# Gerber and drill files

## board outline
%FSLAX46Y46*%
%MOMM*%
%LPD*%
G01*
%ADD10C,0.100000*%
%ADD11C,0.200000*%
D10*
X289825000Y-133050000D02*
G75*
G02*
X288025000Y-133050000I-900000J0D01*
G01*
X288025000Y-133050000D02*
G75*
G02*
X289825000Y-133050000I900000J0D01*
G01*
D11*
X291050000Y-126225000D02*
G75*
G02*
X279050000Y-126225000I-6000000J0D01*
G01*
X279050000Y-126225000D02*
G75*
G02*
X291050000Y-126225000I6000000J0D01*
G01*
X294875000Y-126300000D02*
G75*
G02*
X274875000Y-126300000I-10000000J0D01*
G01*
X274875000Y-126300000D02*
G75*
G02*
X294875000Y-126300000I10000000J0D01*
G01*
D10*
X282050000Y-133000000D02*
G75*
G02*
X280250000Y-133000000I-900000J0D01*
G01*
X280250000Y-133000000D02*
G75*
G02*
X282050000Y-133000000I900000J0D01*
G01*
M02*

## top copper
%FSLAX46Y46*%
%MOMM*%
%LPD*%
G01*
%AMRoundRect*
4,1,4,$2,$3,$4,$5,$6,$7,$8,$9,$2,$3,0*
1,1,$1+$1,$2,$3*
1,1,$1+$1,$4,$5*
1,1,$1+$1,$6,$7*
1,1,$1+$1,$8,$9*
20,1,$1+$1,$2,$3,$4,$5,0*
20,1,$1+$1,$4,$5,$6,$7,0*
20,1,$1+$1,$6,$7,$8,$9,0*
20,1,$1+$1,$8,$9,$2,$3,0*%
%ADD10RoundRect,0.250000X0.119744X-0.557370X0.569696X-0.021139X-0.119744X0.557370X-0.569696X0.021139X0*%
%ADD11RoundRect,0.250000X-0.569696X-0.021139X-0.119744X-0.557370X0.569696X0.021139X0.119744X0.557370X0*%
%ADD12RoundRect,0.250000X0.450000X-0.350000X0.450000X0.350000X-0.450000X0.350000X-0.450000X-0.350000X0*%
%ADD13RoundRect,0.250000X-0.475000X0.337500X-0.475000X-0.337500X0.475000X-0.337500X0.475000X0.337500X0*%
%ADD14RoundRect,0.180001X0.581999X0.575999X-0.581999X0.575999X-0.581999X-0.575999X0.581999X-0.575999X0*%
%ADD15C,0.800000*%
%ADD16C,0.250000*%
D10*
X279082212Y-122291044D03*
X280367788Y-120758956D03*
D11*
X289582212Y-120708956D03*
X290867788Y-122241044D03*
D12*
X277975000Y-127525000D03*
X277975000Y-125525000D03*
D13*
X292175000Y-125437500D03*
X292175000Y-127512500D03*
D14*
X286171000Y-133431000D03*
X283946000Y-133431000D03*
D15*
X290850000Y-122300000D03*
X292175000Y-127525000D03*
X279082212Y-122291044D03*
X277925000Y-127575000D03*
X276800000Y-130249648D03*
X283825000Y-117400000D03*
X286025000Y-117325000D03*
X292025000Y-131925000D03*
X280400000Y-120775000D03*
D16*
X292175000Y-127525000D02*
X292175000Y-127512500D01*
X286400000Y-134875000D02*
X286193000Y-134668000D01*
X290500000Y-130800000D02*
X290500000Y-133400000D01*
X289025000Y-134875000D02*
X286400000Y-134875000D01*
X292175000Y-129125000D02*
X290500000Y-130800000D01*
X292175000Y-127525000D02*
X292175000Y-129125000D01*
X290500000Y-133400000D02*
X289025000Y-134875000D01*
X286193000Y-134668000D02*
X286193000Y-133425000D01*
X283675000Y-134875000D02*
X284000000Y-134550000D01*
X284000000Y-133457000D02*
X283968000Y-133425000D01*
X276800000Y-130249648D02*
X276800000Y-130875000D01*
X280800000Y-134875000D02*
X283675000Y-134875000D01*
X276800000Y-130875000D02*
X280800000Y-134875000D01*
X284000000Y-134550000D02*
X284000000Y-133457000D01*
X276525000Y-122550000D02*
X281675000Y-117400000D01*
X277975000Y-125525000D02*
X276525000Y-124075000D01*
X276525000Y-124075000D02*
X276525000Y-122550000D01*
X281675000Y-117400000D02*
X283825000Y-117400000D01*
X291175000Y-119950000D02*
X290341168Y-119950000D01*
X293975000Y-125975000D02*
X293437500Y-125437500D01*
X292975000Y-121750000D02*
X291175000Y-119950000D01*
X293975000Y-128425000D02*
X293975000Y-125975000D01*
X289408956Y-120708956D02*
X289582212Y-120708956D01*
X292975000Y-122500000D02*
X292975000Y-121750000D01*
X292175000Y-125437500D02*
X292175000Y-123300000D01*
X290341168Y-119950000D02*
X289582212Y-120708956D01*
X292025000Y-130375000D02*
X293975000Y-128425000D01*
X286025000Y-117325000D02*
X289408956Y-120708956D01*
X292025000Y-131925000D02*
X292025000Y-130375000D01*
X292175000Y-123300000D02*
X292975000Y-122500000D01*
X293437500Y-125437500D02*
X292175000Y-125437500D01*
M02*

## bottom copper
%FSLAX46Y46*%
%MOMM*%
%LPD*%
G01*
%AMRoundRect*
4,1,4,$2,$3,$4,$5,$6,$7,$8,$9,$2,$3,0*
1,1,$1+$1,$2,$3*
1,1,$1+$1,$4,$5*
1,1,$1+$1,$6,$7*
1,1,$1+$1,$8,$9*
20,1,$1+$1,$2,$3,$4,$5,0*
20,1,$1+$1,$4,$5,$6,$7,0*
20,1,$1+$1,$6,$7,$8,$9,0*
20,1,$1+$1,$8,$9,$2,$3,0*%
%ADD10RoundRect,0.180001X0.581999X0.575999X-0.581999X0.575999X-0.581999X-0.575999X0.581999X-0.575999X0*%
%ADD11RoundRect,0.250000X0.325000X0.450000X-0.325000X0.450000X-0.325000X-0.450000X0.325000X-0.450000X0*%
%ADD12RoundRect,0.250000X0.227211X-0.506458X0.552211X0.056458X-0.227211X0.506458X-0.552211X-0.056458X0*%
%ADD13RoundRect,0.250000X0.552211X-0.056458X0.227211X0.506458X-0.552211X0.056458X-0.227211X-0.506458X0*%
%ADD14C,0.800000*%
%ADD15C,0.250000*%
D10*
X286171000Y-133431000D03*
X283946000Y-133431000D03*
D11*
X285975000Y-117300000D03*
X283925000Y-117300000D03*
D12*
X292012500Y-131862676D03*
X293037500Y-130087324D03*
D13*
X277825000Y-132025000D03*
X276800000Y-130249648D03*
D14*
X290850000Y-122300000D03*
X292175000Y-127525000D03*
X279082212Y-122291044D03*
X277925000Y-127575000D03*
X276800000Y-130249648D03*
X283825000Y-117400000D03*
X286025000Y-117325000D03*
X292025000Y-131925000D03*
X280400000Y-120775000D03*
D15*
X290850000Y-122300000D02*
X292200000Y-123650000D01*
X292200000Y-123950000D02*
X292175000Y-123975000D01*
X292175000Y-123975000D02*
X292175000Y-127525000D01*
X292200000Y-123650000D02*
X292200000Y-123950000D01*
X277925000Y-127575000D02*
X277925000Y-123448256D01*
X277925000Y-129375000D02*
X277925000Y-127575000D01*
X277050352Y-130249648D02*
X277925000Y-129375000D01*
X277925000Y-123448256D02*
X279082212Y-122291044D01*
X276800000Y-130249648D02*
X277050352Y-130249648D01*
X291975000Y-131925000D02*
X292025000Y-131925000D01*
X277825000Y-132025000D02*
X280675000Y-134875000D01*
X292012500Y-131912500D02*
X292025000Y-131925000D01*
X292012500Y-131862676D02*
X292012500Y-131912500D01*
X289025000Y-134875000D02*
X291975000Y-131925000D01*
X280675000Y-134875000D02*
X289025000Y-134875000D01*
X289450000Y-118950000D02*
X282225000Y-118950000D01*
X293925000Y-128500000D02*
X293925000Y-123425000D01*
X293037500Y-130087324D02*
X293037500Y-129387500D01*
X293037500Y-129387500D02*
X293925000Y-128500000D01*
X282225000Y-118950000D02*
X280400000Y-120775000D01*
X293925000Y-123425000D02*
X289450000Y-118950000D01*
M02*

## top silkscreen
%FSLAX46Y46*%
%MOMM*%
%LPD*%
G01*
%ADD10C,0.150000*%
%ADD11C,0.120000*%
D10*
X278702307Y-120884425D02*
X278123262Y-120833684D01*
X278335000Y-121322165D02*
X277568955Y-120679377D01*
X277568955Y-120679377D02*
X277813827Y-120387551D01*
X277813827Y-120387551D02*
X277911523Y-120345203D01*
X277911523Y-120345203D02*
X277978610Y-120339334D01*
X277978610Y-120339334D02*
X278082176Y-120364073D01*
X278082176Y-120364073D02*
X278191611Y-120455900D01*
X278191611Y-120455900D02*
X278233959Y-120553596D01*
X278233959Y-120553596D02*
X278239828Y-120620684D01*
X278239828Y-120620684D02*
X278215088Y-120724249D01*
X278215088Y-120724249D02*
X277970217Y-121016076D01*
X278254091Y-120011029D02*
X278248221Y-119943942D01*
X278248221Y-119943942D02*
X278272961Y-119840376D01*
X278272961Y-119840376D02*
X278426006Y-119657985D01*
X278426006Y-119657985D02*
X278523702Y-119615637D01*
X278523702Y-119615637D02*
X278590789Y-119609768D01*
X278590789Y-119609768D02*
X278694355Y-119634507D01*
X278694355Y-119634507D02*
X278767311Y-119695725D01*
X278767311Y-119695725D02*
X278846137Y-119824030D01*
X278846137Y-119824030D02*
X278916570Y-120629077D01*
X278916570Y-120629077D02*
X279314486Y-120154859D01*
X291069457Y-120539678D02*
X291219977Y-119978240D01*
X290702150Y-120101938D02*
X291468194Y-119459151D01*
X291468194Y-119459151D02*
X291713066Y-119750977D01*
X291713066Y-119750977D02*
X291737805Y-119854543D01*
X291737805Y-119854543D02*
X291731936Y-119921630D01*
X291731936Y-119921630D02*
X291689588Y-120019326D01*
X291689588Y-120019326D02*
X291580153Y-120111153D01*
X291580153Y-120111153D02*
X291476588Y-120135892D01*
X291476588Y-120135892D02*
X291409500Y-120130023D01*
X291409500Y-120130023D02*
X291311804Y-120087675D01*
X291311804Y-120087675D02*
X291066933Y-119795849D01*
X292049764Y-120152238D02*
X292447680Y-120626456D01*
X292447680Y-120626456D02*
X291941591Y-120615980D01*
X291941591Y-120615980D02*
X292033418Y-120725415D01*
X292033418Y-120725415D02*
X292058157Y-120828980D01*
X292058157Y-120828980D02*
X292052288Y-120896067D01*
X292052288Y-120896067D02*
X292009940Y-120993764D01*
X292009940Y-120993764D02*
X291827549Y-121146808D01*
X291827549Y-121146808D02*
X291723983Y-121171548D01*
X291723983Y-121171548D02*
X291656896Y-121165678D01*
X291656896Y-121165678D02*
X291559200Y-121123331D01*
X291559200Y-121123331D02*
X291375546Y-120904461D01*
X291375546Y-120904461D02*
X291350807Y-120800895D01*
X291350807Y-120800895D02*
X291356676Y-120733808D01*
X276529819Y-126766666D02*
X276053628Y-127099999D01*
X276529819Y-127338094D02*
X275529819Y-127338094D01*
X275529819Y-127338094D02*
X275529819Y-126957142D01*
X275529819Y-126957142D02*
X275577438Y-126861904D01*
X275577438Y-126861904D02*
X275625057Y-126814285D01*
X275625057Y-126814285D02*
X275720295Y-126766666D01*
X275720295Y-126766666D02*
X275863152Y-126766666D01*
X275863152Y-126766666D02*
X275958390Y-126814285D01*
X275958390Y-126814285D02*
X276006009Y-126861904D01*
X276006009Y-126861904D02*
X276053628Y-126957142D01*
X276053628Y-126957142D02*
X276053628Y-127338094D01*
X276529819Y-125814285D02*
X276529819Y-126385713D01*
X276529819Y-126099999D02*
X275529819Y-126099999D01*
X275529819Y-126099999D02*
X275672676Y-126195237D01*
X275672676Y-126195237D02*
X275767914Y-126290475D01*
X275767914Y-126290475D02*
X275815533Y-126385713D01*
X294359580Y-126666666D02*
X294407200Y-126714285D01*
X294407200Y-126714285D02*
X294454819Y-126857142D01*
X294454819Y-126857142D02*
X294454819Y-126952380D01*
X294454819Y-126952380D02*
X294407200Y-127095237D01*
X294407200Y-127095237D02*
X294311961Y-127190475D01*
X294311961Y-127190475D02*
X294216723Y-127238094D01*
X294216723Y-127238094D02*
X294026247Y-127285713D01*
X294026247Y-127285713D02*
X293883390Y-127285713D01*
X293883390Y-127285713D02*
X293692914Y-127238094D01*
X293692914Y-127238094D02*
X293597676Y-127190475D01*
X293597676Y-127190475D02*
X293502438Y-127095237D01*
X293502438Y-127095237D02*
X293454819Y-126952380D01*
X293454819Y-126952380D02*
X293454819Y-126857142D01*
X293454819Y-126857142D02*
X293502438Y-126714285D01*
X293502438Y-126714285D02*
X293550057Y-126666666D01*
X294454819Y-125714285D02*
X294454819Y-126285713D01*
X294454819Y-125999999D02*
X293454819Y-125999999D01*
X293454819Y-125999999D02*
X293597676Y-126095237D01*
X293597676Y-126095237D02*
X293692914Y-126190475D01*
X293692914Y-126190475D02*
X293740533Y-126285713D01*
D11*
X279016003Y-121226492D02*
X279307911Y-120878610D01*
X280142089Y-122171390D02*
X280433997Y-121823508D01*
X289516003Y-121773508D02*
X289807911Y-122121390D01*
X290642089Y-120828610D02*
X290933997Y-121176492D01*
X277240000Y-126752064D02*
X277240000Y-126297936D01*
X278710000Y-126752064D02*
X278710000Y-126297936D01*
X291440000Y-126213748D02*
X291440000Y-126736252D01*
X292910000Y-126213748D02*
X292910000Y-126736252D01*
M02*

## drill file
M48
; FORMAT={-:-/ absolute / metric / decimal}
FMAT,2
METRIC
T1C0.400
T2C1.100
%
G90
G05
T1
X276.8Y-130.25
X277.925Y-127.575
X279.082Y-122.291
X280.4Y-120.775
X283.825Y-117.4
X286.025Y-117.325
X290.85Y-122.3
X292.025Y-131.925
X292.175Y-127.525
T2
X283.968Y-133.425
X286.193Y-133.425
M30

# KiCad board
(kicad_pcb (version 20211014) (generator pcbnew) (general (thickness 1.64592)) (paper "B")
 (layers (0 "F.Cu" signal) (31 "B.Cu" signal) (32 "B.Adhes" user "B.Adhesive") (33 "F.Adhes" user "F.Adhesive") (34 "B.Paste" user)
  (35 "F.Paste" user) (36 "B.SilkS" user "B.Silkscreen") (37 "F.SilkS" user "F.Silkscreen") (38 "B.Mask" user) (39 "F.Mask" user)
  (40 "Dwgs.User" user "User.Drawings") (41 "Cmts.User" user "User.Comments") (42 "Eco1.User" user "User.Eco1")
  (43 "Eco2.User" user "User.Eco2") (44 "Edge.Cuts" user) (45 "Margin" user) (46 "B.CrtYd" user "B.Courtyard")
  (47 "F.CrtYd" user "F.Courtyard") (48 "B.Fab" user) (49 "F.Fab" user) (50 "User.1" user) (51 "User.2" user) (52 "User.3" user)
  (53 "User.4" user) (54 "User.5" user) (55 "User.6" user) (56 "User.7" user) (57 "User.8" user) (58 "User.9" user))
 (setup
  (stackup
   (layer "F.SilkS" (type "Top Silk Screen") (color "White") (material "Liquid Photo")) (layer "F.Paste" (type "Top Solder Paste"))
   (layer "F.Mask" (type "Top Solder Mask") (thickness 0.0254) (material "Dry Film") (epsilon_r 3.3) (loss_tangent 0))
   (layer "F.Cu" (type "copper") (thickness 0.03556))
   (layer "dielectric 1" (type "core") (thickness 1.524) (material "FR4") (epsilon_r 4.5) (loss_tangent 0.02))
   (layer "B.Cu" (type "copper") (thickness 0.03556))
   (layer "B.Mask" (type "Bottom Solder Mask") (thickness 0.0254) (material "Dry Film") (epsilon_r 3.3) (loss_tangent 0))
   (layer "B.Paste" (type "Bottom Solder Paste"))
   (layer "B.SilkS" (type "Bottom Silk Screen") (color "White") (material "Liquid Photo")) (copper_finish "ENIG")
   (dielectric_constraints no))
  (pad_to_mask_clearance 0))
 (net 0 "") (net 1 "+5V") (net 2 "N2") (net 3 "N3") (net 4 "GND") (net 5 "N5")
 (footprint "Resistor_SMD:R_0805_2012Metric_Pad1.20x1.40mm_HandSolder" (layer "F.Cu") (at 279.725 121.525 50)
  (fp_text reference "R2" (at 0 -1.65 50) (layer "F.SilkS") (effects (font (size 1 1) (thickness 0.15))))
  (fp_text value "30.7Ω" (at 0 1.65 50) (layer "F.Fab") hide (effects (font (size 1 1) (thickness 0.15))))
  (fp_line (start -0.227064 -0.735) (end 0.227064 -0.735) (layer "F.SilkS") (width 0.12))
  (fp_line (start -0.227064 0.735) (end 0.227064 0.735) (layer "F.SilkS") (width 0.12))
  (pad "1" smd roundrect (at -1 0 50) (size 1.2 1.4) (layers "F.Cu" "F.Paste" "F.Mask") (roundrect_rratio 0.208333) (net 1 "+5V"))
  (pad "2" smd roundrect (at 1 0 50) (size 1.2 1.4) (layers "F.Cu" "F.Paste" "F.Mask") (roundrect_rratio 0.208333) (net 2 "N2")))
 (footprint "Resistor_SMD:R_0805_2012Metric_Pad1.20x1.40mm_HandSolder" (layer "F.Cu") (at 290.225 121.475 -50)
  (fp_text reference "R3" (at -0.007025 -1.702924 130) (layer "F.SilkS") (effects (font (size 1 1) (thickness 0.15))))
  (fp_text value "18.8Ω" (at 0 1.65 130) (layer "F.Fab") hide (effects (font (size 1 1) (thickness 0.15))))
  (fp_line (start -0.227064 0.735) (end 0.227064 0.735) (layer "F.SilkS") (width 0.12))
  (fp_line (start -0.227064 -0.735) (end 0.227064 -0.735) (layer "F.SilkS") (width 0.12))
  (pad "1" smd roundrect (at -1 0 310) (size 1.2 1.4) (layers "F.Cu" "F.Paste" "F.Mask") (roundrect_rratio 0.208333) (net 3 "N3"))
  (pad "2" smd roundrect (at 1 0 310) (size 1.2 1.4) (layers "F.Cu" "F.Paste" "F.Mask") (roundrect_rratio 0.208333) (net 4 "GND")))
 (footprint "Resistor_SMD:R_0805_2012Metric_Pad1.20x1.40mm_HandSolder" (layer "F.Cu") (at 277.975 126.525 90)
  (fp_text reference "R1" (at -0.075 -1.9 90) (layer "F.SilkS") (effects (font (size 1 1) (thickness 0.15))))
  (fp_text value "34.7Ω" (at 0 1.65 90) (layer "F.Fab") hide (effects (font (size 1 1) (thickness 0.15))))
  (fp_line (start -0.227064 -0.735) (end 0.227064 -0.735) (layer "F.SilkS") (width 0.12))
  (fp_line (start -0.227064 0.735) (end 0.227064 0.735) (layer "F.SilkS") (width 0.12))
  (pad "1" smd roundrect (at -1 0 90) (size 1.2 1.4) (layers "F.Cu" "F.Paste" "F.Mask") (roundrect_rratio 0.208333) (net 1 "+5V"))
  (pad "2" smd roundrect (at 1 0 90) (size 1.2 1.4) (layers "F.Cu" "F.Paste" "F.Mask") (roundrect_rratio 0.208333) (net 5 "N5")))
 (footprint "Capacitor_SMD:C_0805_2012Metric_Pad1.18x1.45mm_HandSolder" (layer "F.Cu") (at 292.175 126.475 -90)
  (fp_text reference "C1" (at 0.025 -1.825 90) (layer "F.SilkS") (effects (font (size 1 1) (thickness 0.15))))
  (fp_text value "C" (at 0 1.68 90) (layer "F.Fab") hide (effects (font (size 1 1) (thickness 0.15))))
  (fp_line (start -0.261252 0.735) (end 0.261252 0.735) (layer "F.SilkS") (width 0.12))
  (fp_line (start -0.261252 -0.735) (end 0.261252 -0.735) (layer "F.SilkS") (width 0.12))
  (pad "1" smd roundrect (at -1.0375 0 270) (size 1.175 1.45) (layers "F.Cu" "F.Paste" "F.Mask") (roundrect_rratio 0.212766) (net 3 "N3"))
  (pad "2" smd roundrect (at 1.0375 0 270) (size 1.175 1.45) (layers "F.Cu" "F.Paste" "F.Mask") (roundrect_rratio 0.212766) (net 4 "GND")))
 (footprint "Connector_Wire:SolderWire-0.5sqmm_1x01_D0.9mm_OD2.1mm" (layer "B.Cu") (at 286.425 133.425 180)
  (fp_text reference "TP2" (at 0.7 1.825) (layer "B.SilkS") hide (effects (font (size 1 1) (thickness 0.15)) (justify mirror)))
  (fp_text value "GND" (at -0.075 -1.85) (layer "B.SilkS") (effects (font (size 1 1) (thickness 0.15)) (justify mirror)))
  (pad "1" thru_hole roundrect (at 0.232 0 180) (size 1.524 1.512) (drill 1.1 (offset 0.022 -0.006)) (layers *.Cu *.Mask)
   (roundrect_rratio 0.119048) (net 4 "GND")))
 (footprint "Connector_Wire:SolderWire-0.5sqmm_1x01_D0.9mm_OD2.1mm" (layer "B.Cu") (at 284.2 133.425 180)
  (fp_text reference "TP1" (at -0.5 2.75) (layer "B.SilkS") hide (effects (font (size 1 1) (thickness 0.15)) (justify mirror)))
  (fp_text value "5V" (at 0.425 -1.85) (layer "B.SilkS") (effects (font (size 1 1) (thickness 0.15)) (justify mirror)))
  (pad "1" thru_hole roundrect (at 0.232 0 180) (size 1.524 1.512) (drill 1.1 (offset 0.022 -0.006)) (layers *.Cu *.Mask)
   (roundrect_rratio 0.119048) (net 1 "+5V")))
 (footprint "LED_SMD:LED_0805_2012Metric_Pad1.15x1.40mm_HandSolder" (layer "B.Cu") (at 284.95 117.3 180)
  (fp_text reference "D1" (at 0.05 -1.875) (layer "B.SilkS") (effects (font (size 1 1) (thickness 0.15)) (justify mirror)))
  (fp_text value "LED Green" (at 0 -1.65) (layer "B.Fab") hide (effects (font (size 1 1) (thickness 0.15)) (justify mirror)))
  (pad "1" smd roundrect (at -1.025 0 180) (size 1.15 1.4) (layers "B.Cu" "B.Paste" "B.Mask") (roundrect_rratio 0.217391) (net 3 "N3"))
  (pad "2" smd roundrect (at 1.025 0 180) (size 1.15 1.4) (layers "B.Cu" "B.Paste" "B.Mask") (roundrect_rratio 0.217391) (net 5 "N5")))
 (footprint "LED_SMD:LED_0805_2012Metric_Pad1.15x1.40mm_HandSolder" (layer "B.Cu") (at 292.525 130.975 60)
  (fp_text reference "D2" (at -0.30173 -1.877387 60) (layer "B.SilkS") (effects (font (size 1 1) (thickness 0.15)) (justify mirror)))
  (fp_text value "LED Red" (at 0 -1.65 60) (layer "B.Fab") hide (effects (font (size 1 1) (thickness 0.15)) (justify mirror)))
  (pad "1" smd roundrect (at -1.025 0 60) (size 1.15 1.4) (layers "B.Cu" "B.Paste" "B.Mask") (roundrect_rratio 0.217391) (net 3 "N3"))
  (pad "2" smd roundrect (at 1.025 0 60) (size 1.15 1.4) (layers "B.Cu" "B.Paste" "B.Mask") (roundrect_rratio 0.217391) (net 2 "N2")))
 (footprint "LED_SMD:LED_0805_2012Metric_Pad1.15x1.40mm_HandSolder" (layer "B.Cu") (at 277.3125 131.137324 120)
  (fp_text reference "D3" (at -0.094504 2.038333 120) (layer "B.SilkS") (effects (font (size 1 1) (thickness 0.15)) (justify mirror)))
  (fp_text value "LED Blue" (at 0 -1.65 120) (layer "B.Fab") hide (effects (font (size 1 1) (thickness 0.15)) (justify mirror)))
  (pad "1" smd roundrect (at -1.025 0 120) (size 1.15 1.4) (layers "B.Cu" "B.Paste" "B.Mask") (roundrect_rratio 0.217391) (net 3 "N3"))
  (pad "2" smd roundrect (at 1.025 0 120) (size 1.15 1.4) (layers "B.Cu" "B.Paste" "B.Mask") (roundrect_rratio 0.217391) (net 1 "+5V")))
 (gr_circle (center 288.925 133.05) (end 289.825 133.05) (layer "Edge.Cuts") (width 0.1) (fill none))
 (gr_circle (center 285.05 126.225) (end 291.05 126.225) (layer "Edge.Cuts") (width 0.2) (fill none))
 (gr_circle (center 284.875 126.3) (end 294.875 126.3) (layer "Edge.Cuts") (width 0.2) (fill none))
 (gr_circle (center 281.15 133) (end 282.05 133) (layer "Edge.Cuts") (width 0.1) (fill none))
 (segment (start 292.175 127.525) (end 292.175 127.5125) (width 0.25) (layer "F.Cu") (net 4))
 (segment (start 286.4 134.875) (end 286.193 134.668) (width 0.25) (layer "F.Cu") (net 4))
 (segment (start 290.5 130.8) (end 290.5 133.4) (width 0.25) (layer "F.Cu") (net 4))
 (segment (start 289.025 134.875) (end 286.4 134.875) (width 0.25) (layer "F.Cu") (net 4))
 (segment (start 292.175 129.125) (end 290.5 130.8) (width 0.25) (layer "F.Cu") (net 4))
 (segment (start 292.175 127.525) (end 292.175 129.125) (width 0.25) (layer "F.Cu") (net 4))
 (segment (start 290.5 133.4) (end 289.025 134.875) (width 0.25) (layer "F.Cu") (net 4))
 (segment (start 286.193 134.668) (end 286.193 133.425) (width 0.25) (layer "F.Cu") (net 4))
 (via (at 290.85 122.3) (size 0.8) (drill 0.4) (layers "F.Cu" "B.Cu") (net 4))
 (via (at 292.175 127.525) (size 0.8) (drill 0.4) (layers "F.Cu" "B.Cu") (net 4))
 (segment (start 290.85 122.3) (end 292.2 123.65) (width 0.25) (layer "B.Cu") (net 4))
 (segment (start 292.2 123.95) (end 292.175 123.975) (width 0.25) (layer "B.Cu") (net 4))
 (segment (start 292.175 123.975) (end 292.175 127.525) (width 0.25) (layer "B.Cu") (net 4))
 (segment (start 292.2 123.65) (end 292.2 123.95) (width 0.25) (layer "B.Cu") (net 4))
 (segment (start 283.675 134.875) (end 284 134.55) (width 0.25) (layer "F.Cu") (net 1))
 (segment (start 284 133.457) (end 283.968 133.425) (width 0.25) (layer "F.Cu") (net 1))
 (segment (start 276.8 130.249648) (end 276.8 130.875) (width 0.25) (layer "F.Cu") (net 1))
 (segment (start 280.8 134.875) (end 283.675 134.875) (width 0.25) (layer "F.Cu") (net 1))
 (segment (start 276.8 130.875) (end 280.8 134.875) (width 0.25) (layer "F.Cu") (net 1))
 (segment (start 284 134.55) (end 284 133.457) (width 0.25) (layer "F.Cu") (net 1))
 (via (at 279.082212 122.291044) (size 0.8) (drill 0.4) (layers "F.Cu" "B.Cu") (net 1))
 (via (at 277.925 127.575) (size 0.8) (drill 0.4) (layers "F.Cu" "B.Cu") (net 1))
 (via (at 276.8 130.249648) (size 0.8) (drill 0.4) (layers "F.Cu" "B.Cu") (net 1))
 (segment (start 277.925 127.575) (end 277.925 123.448256) (width 0.25) (layer "B.Cu") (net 1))
 (segment (start 277.925 129.375) (end 277.925 127.575) (width 0.25) (layer "B.Cu") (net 1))
 (segment (start 277.050352 130.249648) (end 277.925 129.375) (width 0.25) (layer "B.Cu") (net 1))
 (segment (start 277.925 123.448256) (end 279.082212 122.291044) (width 0.25) (layer "B.Cu") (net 1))
 (segment (start 276.8 130.249648) (end 277.050352 130.249648) (width 0.25) (layer "B.Cu") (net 1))
 (segment (start 276.525 122.55) (end 281.675 117.4) (width 0.25) (layer "F.Cu") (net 5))
 (segment (start 277.975 125.525) (end 276.525 124.075) (width 0.25) (layer "F.Cu") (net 5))
 (segment (start 276.525 124.075) (end 276.525 122.55) (width 0.25) (layer "F.Cu") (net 5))
 (segment (start 281.675 117.4) (end 283.825 117.4) (width 0.25) (layer "F.Cu") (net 5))
 (via (at 283.825 117.4) (size 0.8) (drill 0.4) (layers "F.Cu" "B.Cu") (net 5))
 (segment (start 291.175 119.95) (end 290.341168 119.95) (width 0.25) (layer "F.Cu") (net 3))
 (segment (start 293.975 125.975) (end 293.4375 125.4375) (width 0.25) (layer "F.Cu") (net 3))
 (segment (start 292.975 121.75) (end 291.175 119.95) (width 0.25) (layer "F.Cu") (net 3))
 (segment (start 293.975 128.425) (end 293.975 125.975) (width 0.25) (layer "F.Cu") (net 3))
 (segment (start 289.408956 120.708956) (end 289.582212 120.708956) (width 0.25) (layer "F.Cu") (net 3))
 (segment (start 292.975 122.5) (end 292.975 121.75) (width 0.25) (layer "F.Cu") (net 3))
 (segment (start 292.175 125.4375) (end 292.175 123.3) (width 0.25) (layer "F.Cu") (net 3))
 (segment (start 290.341168 119.95) (end 289.582212 120.708956) (width 0.25) (layer "F.Cu") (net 3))
 (segment (start 292.025 130.375) (end 293.975 128.425) (width 0.25) (layer "F.Cu") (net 3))
 (segment (start 286.025 117.325) (end 289.408956 120.708956) (width 0.25) (layer "F.Cu") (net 3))
 (segment (start 292.025 131.925) (end 292.025 130.375) (width 0.25) (layer "F.Cu") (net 3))
 (segment (start 292.175 123.3) (end 292.975 122.5) (width 0.25) (layer "F.Cu") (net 3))
 (segment (start 293.4375 125.4375) (end 292.175 125.4375) (width 0.25) (layer "F.Cu") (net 3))
 (via (at 286.025 117.325) (size 0.8) (drill 0.4) (layers "F.Cu" "B.Cu") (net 3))
 (via (at 292.025 131.925) (size 0.8) (drill 0.4) (layers "F.Cu" "B.Cu") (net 3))
 (segment (start 291.975 131.925) (end 292.025 131.925) (width 0.25) (layer "B.Cu") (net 3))
 (segment (start 277.825 132.025) (end 280.675 134.875) (width 0.25) (layer "B.Cu") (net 3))
 (segment (start 292.0125 131.9125) (end 292.025 131.925) (width 0.25) (layer "B.Cu") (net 3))
 (segment (start 292.0125 131.862676) (end 292.0125 131.9125) (width 0.25) (layer "B.Cu") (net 3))
 (segment (start 289.025 134.875) (end 291.975 131.925) (width 0.25) (layer "B.Cu") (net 3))
 (segment (start 280.675 134.875) (end 289.025 134.875) (width 0.25) (layer "B.Cu") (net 3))
 (via (at 280.4 120.775) (size 0.8) (drill 0.4) (layers "F.Cu" "B.Cu") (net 2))
 (segment (start 289.45 118.95) (end 282.225 118.95) (width 0.25) (layer "B.Cu") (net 2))
 (segment (start 293.925 128.5) (end 293.925 123.425) (width 0.25) (layer "B.Cu") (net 2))
 (segment (start 293.0375 130.087324) (end 293.0375 129.3875) (width 0.25) (layer "B.Cu") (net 2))
 (segment (start 293.0375 129.3875) (end 293.925 128.5) (width 0.25) (layer "B.Cu") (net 2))
 (segment (start 282.225 118.95) (end 280.4 120.775) (width 0.25) (layer "B.Cu") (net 2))
 (segment (start 293.925 123.425) (end 289.45 118.95) (width 0.25) (layer "B.Cu") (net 2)))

